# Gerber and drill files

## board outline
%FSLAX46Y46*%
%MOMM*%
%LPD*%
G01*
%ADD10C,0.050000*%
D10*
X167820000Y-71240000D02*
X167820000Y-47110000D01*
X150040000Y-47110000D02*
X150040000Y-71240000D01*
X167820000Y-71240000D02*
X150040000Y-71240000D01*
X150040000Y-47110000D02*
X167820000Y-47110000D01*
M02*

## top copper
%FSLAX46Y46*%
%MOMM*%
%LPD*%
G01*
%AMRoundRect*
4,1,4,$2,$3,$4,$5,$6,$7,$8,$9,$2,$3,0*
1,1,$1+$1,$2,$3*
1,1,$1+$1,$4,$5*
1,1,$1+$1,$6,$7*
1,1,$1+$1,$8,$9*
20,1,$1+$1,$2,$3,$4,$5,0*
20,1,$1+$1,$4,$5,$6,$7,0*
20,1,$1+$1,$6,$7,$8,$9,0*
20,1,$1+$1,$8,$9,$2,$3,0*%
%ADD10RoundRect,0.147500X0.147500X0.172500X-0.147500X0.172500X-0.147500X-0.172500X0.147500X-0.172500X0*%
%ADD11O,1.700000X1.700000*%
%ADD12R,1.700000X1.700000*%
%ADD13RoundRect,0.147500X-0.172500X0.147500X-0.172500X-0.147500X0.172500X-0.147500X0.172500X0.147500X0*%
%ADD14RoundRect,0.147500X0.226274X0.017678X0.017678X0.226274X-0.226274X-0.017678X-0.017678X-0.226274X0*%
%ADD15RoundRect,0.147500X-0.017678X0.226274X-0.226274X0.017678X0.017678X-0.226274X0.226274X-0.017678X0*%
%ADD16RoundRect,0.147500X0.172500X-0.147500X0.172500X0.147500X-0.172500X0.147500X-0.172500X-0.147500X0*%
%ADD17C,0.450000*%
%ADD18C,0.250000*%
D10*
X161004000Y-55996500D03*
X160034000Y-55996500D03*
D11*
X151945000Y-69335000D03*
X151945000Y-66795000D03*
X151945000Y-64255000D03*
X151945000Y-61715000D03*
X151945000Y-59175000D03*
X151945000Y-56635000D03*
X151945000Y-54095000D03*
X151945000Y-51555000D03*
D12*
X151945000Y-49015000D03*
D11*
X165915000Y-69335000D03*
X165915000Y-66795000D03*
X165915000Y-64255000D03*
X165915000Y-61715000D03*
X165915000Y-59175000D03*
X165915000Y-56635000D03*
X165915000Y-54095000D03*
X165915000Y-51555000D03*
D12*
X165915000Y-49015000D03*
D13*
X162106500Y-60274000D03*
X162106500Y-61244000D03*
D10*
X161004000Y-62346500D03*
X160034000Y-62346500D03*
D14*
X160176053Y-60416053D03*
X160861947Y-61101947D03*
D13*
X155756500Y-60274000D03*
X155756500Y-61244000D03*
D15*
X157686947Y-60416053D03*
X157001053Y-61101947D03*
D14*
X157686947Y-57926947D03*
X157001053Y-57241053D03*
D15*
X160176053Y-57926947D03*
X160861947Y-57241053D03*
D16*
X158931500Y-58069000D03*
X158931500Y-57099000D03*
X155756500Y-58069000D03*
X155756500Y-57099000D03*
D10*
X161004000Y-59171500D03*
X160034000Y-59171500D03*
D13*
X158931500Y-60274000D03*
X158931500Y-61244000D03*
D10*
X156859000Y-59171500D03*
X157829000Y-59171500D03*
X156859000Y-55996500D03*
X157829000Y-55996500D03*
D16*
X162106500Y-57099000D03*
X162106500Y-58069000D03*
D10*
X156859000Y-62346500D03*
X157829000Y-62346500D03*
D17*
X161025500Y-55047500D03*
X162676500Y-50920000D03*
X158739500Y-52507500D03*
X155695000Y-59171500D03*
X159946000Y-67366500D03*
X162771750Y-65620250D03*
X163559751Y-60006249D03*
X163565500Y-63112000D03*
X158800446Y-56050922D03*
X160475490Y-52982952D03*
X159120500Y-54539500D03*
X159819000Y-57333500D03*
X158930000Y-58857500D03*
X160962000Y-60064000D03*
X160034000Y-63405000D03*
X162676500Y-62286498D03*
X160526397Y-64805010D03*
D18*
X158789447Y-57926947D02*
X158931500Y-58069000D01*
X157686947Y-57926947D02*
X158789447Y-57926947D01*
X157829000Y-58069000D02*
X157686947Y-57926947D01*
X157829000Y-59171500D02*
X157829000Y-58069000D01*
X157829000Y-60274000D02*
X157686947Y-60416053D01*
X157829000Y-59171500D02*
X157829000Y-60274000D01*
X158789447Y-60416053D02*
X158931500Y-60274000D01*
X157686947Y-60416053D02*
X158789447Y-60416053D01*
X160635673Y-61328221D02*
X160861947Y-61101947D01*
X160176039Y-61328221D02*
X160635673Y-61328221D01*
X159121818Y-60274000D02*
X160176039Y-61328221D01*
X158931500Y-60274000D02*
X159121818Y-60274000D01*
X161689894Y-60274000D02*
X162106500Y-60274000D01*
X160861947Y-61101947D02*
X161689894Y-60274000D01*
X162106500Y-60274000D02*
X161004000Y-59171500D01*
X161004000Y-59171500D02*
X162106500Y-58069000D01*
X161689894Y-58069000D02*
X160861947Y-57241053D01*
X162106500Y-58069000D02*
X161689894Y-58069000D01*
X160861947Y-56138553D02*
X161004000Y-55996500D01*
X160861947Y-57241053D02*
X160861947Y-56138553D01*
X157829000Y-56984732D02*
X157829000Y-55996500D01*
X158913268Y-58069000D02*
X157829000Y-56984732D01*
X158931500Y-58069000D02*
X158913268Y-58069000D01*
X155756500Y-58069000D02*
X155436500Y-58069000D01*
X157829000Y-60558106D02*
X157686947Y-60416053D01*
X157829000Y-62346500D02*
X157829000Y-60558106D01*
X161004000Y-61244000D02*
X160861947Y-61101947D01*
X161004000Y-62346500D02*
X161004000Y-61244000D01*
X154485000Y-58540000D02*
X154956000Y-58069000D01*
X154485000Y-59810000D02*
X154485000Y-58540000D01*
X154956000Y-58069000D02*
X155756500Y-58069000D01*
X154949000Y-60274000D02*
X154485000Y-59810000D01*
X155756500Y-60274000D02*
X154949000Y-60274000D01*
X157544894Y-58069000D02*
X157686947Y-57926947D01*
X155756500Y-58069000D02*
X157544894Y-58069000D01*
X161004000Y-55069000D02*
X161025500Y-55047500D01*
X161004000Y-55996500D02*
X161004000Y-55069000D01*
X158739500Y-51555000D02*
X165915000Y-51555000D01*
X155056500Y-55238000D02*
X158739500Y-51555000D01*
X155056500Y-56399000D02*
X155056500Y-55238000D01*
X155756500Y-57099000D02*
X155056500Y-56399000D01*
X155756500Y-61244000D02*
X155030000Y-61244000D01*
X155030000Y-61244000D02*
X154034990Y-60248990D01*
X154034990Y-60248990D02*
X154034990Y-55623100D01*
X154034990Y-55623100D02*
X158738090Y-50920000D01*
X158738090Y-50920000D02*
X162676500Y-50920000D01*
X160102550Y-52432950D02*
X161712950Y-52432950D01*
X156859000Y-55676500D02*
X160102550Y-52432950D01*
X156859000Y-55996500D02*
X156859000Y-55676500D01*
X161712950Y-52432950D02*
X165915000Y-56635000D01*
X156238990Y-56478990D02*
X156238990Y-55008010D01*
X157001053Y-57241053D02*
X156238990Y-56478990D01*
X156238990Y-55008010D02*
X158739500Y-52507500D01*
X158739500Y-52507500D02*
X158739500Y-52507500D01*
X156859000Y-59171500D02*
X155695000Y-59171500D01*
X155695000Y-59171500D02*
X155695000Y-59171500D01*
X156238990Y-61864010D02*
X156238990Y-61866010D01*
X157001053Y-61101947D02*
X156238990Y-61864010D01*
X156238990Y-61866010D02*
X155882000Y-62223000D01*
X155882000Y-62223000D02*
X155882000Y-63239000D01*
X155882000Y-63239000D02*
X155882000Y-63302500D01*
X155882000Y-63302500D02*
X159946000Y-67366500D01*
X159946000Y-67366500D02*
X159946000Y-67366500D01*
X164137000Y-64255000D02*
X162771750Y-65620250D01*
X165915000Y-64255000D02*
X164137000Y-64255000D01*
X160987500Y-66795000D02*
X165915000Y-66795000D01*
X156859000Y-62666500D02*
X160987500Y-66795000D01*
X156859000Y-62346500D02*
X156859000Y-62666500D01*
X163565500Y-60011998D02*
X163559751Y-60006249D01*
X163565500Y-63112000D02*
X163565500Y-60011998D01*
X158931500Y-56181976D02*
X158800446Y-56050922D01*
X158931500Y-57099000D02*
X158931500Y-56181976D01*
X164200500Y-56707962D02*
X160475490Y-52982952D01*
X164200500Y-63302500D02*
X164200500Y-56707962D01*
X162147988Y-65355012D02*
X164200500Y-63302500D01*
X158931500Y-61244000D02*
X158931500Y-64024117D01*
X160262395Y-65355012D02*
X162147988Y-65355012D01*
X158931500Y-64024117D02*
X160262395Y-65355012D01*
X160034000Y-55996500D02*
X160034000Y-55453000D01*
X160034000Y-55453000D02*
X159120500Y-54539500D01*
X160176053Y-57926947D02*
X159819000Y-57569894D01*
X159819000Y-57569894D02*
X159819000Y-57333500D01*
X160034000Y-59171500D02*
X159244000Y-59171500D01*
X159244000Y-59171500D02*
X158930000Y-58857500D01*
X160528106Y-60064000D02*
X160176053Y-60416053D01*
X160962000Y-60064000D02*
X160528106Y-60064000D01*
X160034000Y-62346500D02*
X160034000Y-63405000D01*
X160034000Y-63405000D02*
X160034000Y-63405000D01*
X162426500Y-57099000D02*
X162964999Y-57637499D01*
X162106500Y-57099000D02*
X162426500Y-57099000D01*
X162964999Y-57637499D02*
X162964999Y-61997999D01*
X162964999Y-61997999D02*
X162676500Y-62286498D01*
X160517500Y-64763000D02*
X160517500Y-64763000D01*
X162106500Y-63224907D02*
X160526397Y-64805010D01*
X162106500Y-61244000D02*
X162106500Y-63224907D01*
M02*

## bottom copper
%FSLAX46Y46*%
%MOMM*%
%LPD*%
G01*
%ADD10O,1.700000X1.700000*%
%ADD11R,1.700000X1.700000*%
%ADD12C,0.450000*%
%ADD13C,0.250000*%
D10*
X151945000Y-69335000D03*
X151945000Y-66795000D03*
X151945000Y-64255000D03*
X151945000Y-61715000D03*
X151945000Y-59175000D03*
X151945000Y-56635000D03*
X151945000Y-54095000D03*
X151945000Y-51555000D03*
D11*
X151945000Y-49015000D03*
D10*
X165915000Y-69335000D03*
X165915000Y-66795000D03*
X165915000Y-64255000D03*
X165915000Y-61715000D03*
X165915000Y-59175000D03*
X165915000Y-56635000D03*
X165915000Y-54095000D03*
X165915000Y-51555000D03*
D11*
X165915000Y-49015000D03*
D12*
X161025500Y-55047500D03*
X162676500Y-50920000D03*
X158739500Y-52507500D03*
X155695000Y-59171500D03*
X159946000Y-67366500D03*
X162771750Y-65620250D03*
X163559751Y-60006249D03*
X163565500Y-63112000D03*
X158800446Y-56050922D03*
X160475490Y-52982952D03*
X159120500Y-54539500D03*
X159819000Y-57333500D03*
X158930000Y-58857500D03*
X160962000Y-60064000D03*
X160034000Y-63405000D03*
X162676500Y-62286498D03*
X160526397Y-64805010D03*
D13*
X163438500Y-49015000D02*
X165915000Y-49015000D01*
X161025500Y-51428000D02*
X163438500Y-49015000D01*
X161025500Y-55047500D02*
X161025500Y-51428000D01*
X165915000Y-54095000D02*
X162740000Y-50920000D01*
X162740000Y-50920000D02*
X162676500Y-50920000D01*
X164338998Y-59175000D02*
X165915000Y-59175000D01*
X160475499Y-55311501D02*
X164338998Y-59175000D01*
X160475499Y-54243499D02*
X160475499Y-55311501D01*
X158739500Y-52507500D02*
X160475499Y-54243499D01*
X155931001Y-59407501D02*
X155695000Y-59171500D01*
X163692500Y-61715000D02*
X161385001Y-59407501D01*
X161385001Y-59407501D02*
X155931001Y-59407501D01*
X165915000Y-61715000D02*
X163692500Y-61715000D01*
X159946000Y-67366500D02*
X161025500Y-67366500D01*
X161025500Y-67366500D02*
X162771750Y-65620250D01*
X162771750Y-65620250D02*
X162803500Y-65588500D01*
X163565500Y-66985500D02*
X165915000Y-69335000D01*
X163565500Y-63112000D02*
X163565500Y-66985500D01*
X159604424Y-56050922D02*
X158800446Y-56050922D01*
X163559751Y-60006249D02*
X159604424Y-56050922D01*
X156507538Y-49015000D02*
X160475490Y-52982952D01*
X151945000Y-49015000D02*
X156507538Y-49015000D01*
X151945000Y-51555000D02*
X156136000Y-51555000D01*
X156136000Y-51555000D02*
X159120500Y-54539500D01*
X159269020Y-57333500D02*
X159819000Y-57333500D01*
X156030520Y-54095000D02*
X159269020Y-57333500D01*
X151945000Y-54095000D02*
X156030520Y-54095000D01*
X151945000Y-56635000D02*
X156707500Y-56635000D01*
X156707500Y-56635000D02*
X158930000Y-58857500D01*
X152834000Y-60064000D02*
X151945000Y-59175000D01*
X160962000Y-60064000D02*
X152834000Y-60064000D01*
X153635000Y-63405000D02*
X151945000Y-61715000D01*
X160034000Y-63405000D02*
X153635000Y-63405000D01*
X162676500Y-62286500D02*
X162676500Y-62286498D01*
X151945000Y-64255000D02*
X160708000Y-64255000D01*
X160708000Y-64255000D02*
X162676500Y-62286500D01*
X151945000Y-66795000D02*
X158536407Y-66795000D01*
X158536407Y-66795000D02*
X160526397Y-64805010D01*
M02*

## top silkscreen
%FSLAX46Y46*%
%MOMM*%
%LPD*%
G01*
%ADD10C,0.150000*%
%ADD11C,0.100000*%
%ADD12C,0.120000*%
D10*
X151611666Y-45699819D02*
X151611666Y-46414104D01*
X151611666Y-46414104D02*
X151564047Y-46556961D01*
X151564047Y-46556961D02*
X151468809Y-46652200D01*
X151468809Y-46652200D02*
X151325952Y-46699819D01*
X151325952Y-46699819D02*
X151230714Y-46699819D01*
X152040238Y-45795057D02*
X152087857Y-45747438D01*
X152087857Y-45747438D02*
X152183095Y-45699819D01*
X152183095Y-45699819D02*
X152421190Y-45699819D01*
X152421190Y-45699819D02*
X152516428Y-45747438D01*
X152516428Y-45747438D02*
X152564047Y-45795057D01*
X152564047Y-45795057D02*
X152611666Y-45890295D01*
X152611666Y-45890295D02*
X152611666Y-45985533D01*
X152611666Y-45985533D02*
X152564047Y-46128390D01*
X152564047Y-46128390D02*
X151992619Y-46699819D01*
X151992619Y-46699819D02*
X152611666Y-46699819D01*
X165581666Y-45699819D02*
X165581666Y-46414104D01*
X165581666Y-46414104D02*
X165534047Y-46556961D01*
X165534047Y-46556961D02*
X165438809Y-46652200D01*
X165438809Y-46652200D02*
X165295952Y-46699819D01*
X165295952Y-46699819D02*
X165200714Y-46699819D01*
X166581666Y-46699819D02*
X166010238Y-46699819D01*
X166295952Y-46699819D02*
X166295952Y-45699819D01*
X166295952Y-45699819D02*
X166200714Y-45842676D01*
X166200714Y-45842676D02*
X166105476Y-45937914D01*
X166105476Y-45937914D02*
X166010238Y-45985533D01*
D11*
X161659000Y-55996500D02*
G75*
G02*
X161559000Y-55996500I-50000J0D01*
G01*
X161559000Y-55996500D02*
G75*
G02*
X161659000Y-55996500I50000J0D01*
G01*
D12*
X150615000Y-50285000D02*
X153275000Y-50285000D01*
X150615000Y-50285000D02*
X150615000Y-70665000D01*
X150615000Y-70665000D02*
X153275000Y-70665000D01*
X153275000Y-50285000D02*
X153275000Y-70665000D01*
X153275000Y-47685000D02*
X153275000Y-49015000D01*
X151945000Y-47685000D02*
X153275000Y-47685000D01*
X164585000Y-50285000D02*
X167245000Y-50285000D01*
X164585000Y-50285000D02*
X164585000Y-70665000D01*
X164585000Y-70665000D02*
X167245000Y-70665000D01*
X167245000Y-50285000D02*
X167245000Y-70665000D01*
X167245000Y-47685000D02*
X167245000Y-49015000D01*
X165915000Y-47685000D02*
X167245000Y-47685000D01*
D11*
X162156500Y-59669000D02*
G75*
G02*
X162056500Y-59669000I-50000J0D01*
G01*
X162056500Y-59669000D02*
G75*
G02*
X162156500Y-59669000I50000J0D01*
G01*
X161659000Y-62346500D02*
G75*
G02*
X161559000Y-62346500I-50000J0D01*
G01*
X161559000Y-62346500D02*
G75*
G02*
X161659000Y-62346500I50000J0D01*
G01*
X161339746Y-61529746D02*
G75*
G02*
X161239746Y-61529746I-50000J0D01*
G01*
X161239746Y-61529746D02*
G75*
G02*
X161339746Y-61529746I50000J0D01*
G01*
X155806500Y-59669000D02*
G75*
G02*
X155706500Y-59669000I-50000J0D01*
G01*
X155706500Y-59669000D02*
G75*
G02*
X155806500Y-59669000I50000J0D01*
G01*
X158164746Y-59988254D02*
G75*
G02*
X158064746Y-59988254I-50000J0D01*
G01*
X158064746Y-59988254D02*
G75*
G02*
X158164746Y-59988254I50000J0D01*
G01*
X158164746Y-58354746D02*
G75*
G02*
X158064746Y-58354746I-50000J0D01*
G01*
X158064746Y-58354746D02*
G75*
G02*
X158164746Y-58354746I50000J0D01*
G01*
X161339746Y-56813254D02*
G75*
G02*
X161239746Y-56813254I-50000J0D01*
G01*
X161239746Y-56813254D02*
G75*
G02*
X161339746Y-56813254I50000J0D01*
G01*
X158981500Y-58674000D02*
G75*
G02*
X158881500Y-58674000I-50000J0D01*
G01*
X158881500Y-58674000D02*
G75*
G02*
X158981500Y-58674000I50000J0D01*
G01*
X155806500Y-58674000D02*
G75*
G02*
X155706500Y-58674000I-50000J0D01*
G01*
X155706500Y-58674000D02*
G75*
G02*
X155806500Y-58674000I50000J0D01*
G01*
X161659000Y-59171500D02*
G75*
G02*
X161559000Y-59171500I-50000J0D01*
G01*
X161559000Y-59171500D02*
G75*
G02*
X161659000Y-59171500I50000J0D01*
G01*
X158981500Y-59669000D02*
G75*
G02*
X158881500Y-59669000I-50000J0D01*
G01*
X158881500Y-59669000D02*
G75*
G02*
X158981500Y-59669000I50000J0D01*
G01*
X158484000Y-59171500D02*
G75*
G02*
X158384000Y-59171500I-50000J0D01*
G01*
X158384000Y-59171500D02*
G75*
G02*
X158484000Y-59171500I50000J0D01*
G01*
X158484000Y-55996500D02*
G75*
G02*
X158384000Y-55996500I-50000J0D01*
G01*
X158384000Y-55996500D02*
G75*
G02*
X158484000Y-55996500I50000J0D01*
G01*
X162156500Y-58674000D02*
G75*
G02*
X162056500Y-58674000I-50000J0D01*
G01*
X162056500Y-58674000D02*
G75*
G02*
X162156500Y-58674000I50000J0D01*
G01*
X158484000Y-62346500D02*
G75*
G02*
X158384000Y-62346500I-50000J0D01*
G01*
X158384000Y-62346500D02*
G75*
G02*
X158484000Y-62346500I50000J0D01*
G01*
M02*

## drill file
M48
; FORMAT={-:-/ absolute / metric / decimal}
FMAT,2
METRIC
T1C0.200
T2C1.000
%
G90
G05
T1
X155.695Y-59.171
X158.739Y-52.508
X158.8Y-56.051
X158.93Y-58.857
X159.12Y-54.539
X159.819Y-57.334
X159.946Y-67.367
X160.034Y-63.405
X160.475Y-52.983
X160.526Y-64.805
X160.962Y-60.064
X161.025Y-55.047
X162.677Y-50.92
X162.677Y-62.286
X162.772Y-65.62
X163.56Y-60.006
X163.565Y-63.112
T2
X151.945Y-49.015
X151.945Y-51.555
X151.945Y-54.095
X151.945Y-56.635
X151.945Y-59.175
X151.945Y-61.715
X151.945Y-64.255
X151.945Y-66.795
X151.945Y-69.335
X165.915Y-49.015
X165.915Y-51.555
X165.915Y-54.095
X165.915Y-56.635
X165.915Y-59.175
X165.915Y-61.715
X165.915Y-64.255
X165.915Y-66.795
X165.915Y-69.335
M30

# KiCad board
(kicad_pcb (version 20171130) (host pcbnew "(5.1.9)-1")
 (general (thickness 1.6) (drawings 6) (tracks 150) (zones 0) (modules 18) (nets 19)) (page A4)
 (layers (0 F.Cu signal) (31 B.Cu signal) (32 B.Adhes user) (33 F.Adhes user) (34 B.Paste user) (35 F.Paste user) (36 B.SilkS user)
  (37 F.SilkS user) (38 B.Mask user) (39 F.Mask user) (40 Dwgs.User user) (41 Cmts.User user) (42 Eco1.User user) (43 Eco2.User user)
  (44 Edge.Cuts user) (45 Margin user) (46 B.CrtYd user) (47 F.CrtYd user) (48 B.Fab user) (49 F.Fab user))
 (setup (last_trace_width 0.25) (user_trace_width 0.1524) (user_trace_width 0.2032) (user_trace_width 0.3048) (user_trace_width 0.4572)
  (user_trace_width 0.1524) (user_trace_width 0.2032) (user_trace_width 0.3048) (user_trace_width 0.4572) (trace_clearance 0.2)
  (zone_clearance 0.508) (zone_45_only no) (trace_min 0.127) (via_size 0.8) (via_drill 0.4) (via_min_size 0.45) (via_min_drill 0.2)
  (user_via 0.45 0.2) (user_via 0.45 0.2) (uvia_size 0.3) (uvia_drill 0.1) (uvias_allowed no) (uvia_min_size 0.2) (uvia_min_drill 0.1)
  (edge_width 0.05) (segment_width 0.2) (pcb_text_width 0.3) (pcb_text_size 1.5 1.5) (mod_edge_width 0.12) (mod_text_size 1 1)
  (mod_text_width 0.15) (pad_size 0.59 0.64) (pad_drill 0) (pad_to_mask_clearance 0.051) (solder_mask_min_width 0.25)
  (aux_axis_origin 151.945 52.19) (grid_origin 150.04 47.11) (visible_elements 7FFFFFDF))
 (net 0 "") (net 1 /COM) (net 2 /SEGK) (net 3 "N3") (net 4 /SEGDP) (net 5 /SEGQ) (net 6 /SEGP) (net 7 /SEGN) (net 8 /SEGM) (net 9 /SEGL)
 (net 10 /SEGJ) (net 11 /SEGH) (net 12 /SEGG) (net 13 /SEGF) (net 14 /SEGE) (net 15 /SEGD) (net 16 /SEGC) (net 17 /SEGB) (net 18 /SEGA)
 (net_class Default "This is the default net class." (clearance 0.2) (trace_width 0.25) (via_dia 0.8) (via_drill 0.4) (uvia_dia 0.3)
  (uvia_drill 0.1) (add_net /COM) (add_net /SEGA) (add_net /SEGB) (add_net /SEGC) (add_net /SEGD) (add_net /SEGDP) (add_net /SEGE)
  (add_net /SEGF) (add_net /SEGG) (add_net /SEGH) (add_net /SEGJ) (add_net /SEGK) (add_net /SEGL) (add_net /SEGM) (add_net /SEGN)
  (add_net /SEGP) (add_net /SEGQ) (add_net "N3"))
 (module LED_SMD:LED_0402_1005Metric (layer F.Cu) (at 160.519 55.9965 180)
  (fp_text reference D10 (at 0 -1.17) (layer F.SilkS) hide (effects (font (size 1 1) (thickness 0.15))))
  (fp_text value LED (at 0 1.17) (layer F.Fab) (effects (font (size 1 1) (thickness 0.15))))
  (fp_circle (center -1.09 0) (end -1.04 0) (layer F.SilkS) (width 0.1))
  (pad 1 smd roundrect (at -0.485 0 180) (size 0.59 0.64) (layers F.Cu F.Paste F.Mask) (roundrect_rratio 0.25) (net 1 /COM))
  (pad 2 smd roundrect (at 0.485 0 180) (size 0.59 0.64) (layers F.Cu F.Paste F.Mask) (roundrect_rratio 0.25) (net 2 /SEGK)))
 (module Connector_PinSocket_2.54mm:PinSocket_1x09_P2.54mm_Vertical (layer F.Cu) (at 151.945 49.015)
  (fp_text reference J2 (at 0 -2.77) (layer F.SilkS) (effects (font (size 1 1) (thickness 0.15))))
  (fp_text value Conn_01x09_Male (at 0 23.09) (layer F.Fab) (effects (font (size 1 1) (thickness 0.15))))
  (fp_line (start -1.33 1.27) (end 1.33 1.27) (layer F.SilkS) (width 0.12))
  (fp_line (start -1.33 1.27) (end -1.33 21.65) (layer F.SilkS) (width 0.12))
  (fp_line (start -1.33 21.65) (end 1.33 21.65) (layer F.SilkS) (width 0.12))
  (fp_line (start 1.33 1.27) (end 1.33 21.65) (layer F.SilkS) (width 0.12))
  (fp_line (start 1.33 -1.33) (end 1.33 0) (layer F.SilkS) (width 0.12))
  (fp_line (start 0 -1.33) (end 1.33 -1.33) (layer F.SilkS) (width 0.12))
  (pad 9 thru_hole oval (at 0 20.32) (size 1.7 1.7) (drill 1) (layers *.Cu *.Mask) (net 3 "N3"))
  (pad 8 thru_hole oval (at 0 17.78) (size 1.7 1.7) (drill 1) (layers *.Cu *.Mask) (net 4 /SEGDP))
  (pad 7 thru_hole oval (at 0 15.24) (size 1.7 1.7) (drill 1) (layers *.Cu *.Mask) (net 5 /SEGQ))
  (pad 6 thru_hole oval (at 0 12.7) (size 1.7 1.7) (drill 1) (layers *.Cu *.Mask) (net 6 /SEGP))
  (pad 5 thru_hole oval (at 0 10.16) (size 1.7 1.7) (drill 1) (layers *.Cu *.Mask) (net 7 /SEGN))
  (pad 4 thru_hole oval (at 0 7.62) (size 1.7 1.7) (drill 1) (layers *.Cu *.Mask) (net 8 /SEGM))
  (pad 3 thru_hole oval (at 0 5.08) (size 1.7 1.7) (drill 1) (layers *.Cu *.Mask) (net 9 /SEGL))
  (pad 2 thru_hole oval (at 0 2.54) (size 1.7 1.7) (drill 1) (layers *.Cu *.Mask) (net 2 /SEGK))
  (pad 1 thru_hole rect (at 0 0) (size 1.7 1.7) (drill 1) (layers *.Cu *.Mask) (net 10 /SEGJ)))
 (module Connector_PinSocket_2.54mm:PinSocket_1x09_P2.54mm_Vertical (layer F.Cu) (at 165.915 49.015)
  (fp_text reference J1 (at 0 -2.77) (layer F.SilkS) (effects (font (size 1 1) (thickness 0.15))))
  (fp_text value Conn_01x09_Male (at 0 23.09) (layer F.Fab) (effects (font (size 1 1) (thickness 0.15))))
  (fp_line (start -1.33 1.27) (end 1.33 1.27) (layer F.SilkS) (width 0.12))
  (fp_line (start -1.33 1.27) (end -1.33 21.65) (layer F.SilkS) (width 0.12))
  (fp_line (start -1.33 21.65) (end 1.33 21.65) (layer F.SilkS) (width 0.12))
  (fp_line (start 1.33 1.27) (end 1.33 21.65) (layer F.SilkS) (width 0.12))
  (fp_line (start 1.33 -1.33) (end 1.33 0) (layer F.SilkS) (width 0.12))
  (fp_line (start 0 -1.33) (end 1.33 -1.33) (layer F.SilkS) (width 0.12))
  (pad 9 thru_hole oval (at 0 20.32) (size 1.7 1.7) (drill 1) (layers *.Cu *.Mask) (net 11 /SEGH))
  (pad 8 thru_hole oval (at 0 17.78) (size 1.7 1.7) (drill 1) (layers *.Cu *.Mask) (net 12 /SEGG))
  (pad 7 thru_hole oval (at 0 15.24) (size 1.7 1.7) (drill 1) (layers *.Cu *.Mask) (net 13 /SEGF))
  (pad 6 thru_hole oval (at 0 12.7) (size 1.7 1.7) (drill 1) (layers *.Cu *.Mask) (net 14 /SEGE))
  (pad 5 thru_hole oval (at 0 10.16) (size 1.7 1.7) (drill 1) (layers *.Cu *.Mask) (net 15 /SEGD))
  (pad 4 thru_hole oval (at 0 7.62) (size 1.7 1.7) (drill 1) (layers *.Cu *.Mask) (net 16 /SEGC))
  (pad 3 thru_hole oval (at 0 5.08) (size 1.7 1.7) (drill 1) (layers *.Cu *.Mask) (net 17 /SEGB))
  (pad 2 thru_hole oval (at 0 2.54) (size 1.7 1.7) (drill 1) (layers *.Cu *.Mask) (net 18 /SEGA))
  (pad 1 thru_hole rect (at 0 0) (size 1.7 1.7) (drill 1) (layers *.Cu *.Mask) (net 1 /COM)))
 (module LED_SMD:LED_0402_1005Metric (layer F.Cu) (at 162.1065 60.759 270)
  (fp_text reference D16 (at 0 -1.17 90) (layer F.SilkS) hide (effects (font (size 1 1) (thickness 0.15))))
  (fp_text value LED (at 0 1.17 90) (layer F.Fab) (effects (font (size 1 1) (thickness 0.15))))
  (fp_circle (center -1.09 0) (end -1.04 0) (layer F.SilkS) (width 0.1))
  (pad 1 smd roundrect (at -0.485 0 270) (size 0.59 0.64) (layers F.Cu F.Paste F.Mask) (roundrect_rratio 0.25) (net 1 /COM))
  (pad 2 smd roundrect (at 0.485 0 270) (size 0.59 0.64) (layers F.Cu F.Paste F.Mask) (roundrect_rratio 0.25) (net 4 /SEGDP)))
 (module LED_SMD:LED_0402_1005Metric (layer F.Cu) (at 160.519 62.3465 180)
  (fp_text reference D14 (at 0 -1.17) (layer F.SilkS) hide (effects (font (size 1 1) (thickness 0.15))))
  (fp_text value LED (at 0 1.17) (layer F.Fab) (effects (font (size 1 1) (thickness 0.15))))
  (fp_circle (center -1.09 0) (end -1.04 0) (layer F.SilkS) (width 0.1))
  (pad 1 smd roundrect (at -0.485 0 180) (size 0.59 0.64) (layers F.Cu F.Paste F.Mask) (roundrect_rratio 0.25) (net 1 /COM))
  (pad 2 smd roundrect (at 0.485 0 180) (size 0.59 0.64) (layers F.Cu F.Paste F.Mask) (roundrect_rratio 0.25) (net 6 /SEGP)))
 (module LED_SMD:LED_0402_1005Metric (layer F.Cu) (at 160.519 60.759 135)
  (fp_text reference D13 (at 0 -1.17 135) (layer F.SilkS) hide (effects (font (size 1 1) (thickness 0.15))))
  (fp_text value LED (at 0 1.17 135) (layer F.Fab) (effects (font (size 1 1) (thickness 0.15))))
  (fp_circle (center -1.09 0) (end -1.04 0) (layer F.SilkS) (width 0.1))
  (pad 2 smd roundrect (at 0.485 0 135) (size 0.59 0.64) (layers F.Cu F.Paste F.Mask) (roundrect_rratio 0.25) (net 7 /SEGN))
  (pad 1 smd roundrect (at -0.485 0 135) (size 0.59 0.64) (layers F.Cu F.Paste F.Mask) (roundrect_rratio 0.25) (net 1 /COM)))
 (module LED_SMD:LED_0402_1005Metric (layer F.Cu) (at 155.7565 60.759 270)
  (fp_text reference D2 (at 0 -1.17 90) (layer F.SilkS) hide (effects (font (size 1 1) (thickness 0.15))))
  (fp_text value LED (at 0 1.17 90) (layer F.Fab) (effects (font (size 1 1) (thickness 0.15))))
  (fp_circle (center -1.09 0) (end -1.04 0) (layer F.SilkS) (width 0.1))
  (pad 1 smd roundrect (at -0.485 0 270) (size 0.59 0.64) (layers F.Cu F.Paste F.Mask) (roundrect_rratio 0.25) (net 1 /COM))
  (pad 2 smd roundrect (at 0.485 0 270) (size 0.59 0.64) (layers F.Cu F.Paste F.Mask) (roundrect_rratio 0.25) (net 17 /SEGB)))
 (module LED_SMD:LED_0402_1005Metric (layer F.Cu) (at 157.344 60.759 225)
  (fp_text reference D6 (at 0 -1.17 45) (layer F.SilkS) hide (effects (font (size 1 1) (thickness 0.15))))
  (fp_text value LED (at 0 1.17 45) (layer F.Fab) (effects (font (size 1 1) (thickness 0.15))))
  (fp_circle (center -1.09 0) (end -1.04 0) (layer F.SilkS) (width 0.1))
  (pad 1 smd roundrect (at -0.485 0 225) (size 0.59 0.64) (layers F.Cu F.Paste F.Mask) (roundrect_rratio 0.25) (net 1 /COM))
  (pad 2 smd roundrect (at 0.485 0 225) (size 0.59 0.64) (layers F.Cu F.Paste F.Mask) (roundrect_rratio 0.25) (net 13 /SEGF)))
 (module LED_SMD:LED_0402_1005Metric (layer F.Cu) (at 157.344 57.584 135)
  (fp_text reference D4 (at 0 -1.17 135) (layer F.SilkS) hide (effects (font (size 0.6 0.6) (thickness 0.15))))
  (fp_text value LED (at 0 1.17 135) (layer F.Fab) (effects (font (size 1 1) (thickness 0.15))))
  (fp_circle (center -1.09 0) (end -1.04 0) (layer F.SilkS) (width 0.1))
  (pad 1 smd roundrect (at -0.485 0 135) (size 0.59 0.64) (layers F.Cu F.Paste F.Mask) (roundrect_rratio 0.25) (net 1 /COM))
  (pad 2 smd roundrect (at 0.485 0 135) (size 0.59 0.64) (layers F.Cu F.Paste F.Mask) (roundrect_rratio 0.25) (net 15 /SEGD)))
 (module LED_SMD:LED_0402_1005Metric (layer F.Cu) (at 160.519 57.584 225)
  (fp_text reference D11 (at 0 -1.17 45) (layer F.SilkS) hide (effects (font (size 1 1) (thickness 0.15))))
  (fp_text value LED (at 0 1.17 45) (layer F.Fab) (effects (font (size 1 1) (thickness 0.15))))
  (fp_circle (center -1.09 0) (end -1.04 0) (layer F.SilkS) (width 0.1))
  (pad 2 smd roundrect (at 0.485 0 225) (size 0.59 0.64) (layers F.Cu F.Paste F.Mask) (roundrect_rratio 0.25) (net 9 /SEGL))
  (pad 1 smd roundrect (at -0.485 0 225) (size 0.59 0.64) (layers F.Cu F.Paste F.Mask) (roundrect_rratio 0.25) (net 1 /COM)))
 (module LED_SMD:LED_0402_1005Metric (layer F.Cu) (at 158.9315 57.584 90)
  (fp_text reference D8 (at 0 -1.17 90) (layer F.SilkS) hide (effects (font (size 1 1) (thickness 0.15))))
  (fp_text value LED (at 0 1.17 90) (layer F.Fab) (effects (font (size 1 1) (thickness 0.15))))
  (fp_circle (center -1.09 0) (end -1.04 0) (layer F.SilkS) (width 0.1))
  (pad 1 smd roundrect (at -0.485 0 90) (size 0.59 0.64) (layers F.Cu F.Paste F.Mask) (roundrect_rratio 0.25) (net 1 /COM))
  (pad 2 smd roundrect (at 0.485 0 90) (size 0.59 0.64) (layers F.Cu F.Paste F.Mask) (roundrect_rratio 0.25) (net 11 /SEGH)))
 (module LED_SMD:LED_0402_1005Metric (layer F.Cu) (at 155.7565 57.584 90)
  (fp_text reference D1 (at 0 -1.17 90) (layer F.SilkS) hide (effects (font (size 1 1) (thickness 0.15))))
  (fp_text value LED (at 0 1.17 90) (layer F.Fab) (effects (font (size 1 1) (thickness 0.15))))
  (fp_circle (center -1.09 0) (end -1.04 0) (layer F.SilkS) (width 0.1))
  (pad 1 smd roundrect (at -0.485 0 90) (size 0.59 0.64) (layers F.Cu F.Paste F.Mask) (roundrect_rratio 0.25) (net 1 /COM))
  (pad 2 smd roundrect (at 0.485 0 90) (size 0.59 0.64) (layers F.Cu F.Paste F.Mask) (roundrect_rratio 0.25) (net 18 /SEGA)))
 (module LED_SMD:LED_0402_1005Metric (layer F.Cu) (at 160.519 59.1715 180)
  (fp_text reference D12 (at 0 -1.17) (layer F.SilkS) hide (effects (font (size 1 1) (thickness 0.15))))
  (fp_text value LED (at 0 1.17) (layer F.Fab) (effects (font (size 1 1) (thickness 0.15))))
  (fp_circle (center -1.09 0) (end -1.04 0) (layer F.SilkS) (width 0.1))
  (pad 1 smd roundrect (at -0.485 0 180) (size 0.59 0.64) (layers F.Cu F.Paste F.Mask) (roundrect_rratio 0.25) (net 1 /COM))
  (pad 2 smd roundrect (at 0.485 0 180) (size 0.59 0.64) (layers F.Cu F.Paste F.Mask) (roundrect_rratio 0.25) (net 8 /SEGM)))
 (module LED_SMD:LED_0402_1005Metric (layer F.Cu) (at 158.9315 60.759 270)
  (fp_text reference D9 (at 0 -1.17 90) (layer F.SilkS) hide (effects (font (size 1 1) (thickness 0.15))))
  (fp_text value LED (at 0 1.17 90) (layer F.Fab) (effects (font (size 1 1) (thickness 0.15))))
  (fp_circle (center -1.09 0) (end -1.04 0) (layer F.SilkS) (width 0.1))
  (pad 1 smd roundrect (at -0.485 0 270) (size 0.59 0.64) (layers F.Cu F.Paste F.Mask) (roundrect_rratio 0.25) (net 1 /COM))
  (pad 2 smd roundrect (at 0.485 0 270) (size 0.59 0.64) (layers F.Cu F.Paste F.Mask) (roundrect_rratio 0.25) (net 10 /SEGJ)))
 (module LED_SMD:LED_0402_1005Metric (layer F.Cu) (at 157.344 59.1715 180)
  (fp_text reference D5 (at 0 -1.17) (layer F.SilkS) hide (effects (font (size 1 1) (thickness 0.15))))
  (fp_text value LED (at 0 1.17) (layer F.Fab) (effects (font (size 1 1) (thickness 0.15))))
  (fp_circle (center -1.09 0) (end -1.04 0) (layer F.SilkS) (width 0.1))
  (pad 2 smd roundrect (at 0.485 0 180) (size 0.59 0.64) (layers F.Cu F.Paste F.Mask) (roundrect_rratio 0.25) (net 14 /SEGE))
  (pad 1 smd roundrect (at -0.485 0 180) (size 0.59 0.64) (layers F.Cu F.Paste F.Mask) (roundrect_rratio 0.25) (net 1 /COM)))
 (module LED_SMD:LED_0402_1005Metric (layer F.Cu) (at 157.344 55.9965 180)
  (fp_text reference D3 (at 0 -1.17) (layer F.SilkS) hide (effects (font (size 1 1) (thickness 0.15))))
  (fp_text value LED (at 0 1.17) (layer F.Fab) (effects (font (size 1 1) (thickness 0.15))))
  (fp_circle (center -1.09 0) (end -1.04 0) (layer F.SilkS) (width 0.1))
  (pad 2 smd roundrect (at 0.485 0 180) (size 0.59 0.64) (layers F.Cu F.Paste F.Mask) (roundrect_rratio 0.25) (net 16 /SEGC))
  (pad 1 smd roundrect (at -0.485 0 180) (size 0.59 0.64) (layers F.Cu F.Paste F.Mask) (roundrect_rratio 0.25) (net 1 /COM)))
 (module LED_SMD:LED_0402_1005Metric (layer F.Cu) (at 162.1065 57.584 90)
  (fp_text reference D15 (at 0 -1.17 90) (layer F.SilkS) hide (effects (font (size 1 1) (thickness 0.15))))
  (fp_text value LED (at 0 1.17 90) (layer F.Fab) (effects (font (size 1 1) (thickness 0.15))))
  (fp_circle (center -1.09 0) (end -1.04 0) (layer F.SilkS) (width 0.1))
  (pad 2 smd roundrect (at 0.485 0 90) (size 0.59 0.64) (layers F.Cu F.Paste F.Mask) (roundrect_rratio 0.25) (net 5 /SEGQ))
  (pad 1 smd roundrect (at -0.485 0 90) (size 0.59 0.64) (layers F.Cu F.Paste F.Mask) (roundrect_rratio 0.25) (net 1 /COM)))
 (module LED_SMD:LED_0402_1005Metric (layer F.Cu) (at 157.344 62.3465 180)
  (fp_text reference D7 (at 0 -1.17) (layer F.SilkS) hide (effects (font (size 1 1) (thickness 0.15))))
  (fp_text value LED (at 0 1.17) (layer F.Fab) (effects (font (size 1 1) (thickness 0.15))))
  (fp_circle (center -1.09 0) (end -1.04 0) (layer F.SilkS) (width 0.1))
  (pad 2 smd roundrect (at 0.485 0 180) (size 0.59 0.64) (layers F.Cu F.Paste F.Mask) (roundrect_rratio 0.25) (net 12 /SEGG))
  (pad 1 smd roundrect (at -0.485 0 180) (size 0.59 0.64) (layers F.Cu F.Paste F.Mask) (roundrect_rratio 0.25) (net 1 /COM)))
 (gr_line (start 167.82 71.24) (end 167.82 47.11) (layer Edge.Cuts) (width 0.05))
 (gr_line (start 150.04 47.11) (end 150.04 71.24) (layer Edge.Cuts) (width 0.05))
 (gr_line (start 167.82 71.24) (end 150.04 71.24) (layer Edge.Cuts) (width 0.05))
 (gr_line (start 150.04 47.11) (end 167.82 47.11) (layer Edge.Cuts) (width 0.05))
 (via (at 161.0255 55.0475) (size 0.45) (drill 0.2) (layers F.Cu B.Cu) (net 1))
 (segment (start 158.789447 57.926947) (end 158.9315 58.069) (width 0.25) (layer F.Cu) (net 1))
 (segment (start 157.686947 57.926947) (end 158.789447 57.926947) (width 0.25) (layer F.Cu) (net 1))
 (segment (start 157.829 58.069) (end 157.686947 57.926947) (width 0.25) (layer F.Cu) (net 1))
 (segment (start 157.829 59.1715) (end 157.829 58.069) (width 0.25) (layer F.Cu) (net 1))
 (segment (start 157.829 60.274) (end 157.686947 60.416053) (width 0.25) (layer F.Cu) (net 1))
 (segment (start 157.829 59.1715) (end 157.829 60.274) (width 0.25) (layer F.Cu) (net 1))
 (segment (start 158.789447 60.416053) (end 158.9315 60.274) (width 0.25) (layer F.Cu) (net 1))
 (segment (start 157.686947 60.416053) (end 158.789447 60.416053) (width 0.25) (layer F.Cu) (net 1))
 (segment (start 160.635673 61.328221) (end 160.861947 61.101947) (width 0.25) (layer F.Cu) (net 1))
 (segment (start 160.176039 61.328221) (end 160.635673 61.328221) (width 0.25) (layer F.Cu) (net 1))
 (segment (start 159.121818 60.274) (end 160.176039 61.328221) (width 0.25) (layer F.Cu) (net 1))
 (segment (start 158.9315 60.274) (end 159.121818 60.274) (width 0.25) (layer F.Cu) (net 1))
 (segment (start 161.689894 60.274) (end 162.1065 60.274) (width 0.25) (layer F.Cu) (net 1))
 (segment (start 160.861947 61.101947) (end 161.689894 60.274) (width 0.25) (layer F.Cu) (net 1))
 (segment (start 162.1065 60.274) (end 161.004 59.1715) (width 0.25) (layer F.Cu) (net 1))
 (segment (start 161.004 59.1715) (end 162.1065 58.069) (width 0.25) (layer F.Cu) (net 1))
 (segment (start 161.689894 58.069) (end 160.861947 57.241053) (width 0.25) (layer F.Cu) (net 1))
 (segment (start 162.1065 58.069) (end 161.689894 58.069) (width 0.25) (layer F.Cu) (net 1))
 (segment (start 160.861947 56.138553) (end 161.004 55.9965) (width 0.25) (layer F.Cu) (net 1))
 (segment (start 160.861947 57.241053) (end 160.861947 56.138553) (width 0.25) (layer F.Cu) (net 1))
 (segment (start 157.829 56.984732) (end 157.829 55.9965) (width 0.25) (layer F.Cu) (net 1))
 (segment (start 158.913268 58.069) (end 157.829 56.984732) (width 0.25) (layer F.Cu) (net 1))
 (segment (start 158.9315 58.069) (end 158.913268 58.069) (width 0.25) (layer F.Cu) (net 1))
 (segment (start 155.7565 58.069) (end 155.4365 58.069) (width 0.25) (layer F.Cu) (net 1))
 (segment (start 157.829 60.558106) (end 157.686947 60.416053) (width 0.25) (layer F.Cu) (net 1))
 (segment (start 157.829 62.3465) (end 157.829 60.558106) (width 0.25) (layer F.Cu) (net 1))
 (segment (start 161.004 61.244) (end 160.861947 61.101947) (width 0.25) (layer F.Cu) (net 1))
 (segment (start 161.004 62.3465) (end 161.004 61.244) (width 0.25) (layer F.Cu) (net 1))
 (segment (start 154.485 58.54) (end 154.956 58.069) (width 0.25) (layer F.Cu) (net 1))
 (segment (start 154.485 59.81) (end 154.485 58.54) (width 0.25) (layer F.Cu) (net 1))
 (segment (start 154.956 58.069) (end 155.7565 58.069) (width 0.25) (layer F.Cu) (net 1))
 (segment (start 154.949 60.274) (end 154.485 59.81) (width 0.25) (layer F.Cu) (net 1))
 (segment (start 155.7565 60.274) (end 154.949 60.274) (width 0.25) (layer F.Cu) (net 1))
 (segment (start 157.544894 58.069) (end 157.686947 57.926947) (width 0.25) (layer F.Cu) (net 1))
 (segment (start 155.7565 58.069) (end 157.544894 58.069) (width 0.25) (layer F.Cu) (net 1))
 (segment (start 161.004 55.069) (end 161.0255 55.0475) (width 0.25) (layer F.Cu) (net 1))
 (segment (start 161.004 55.9965) (end 161.004 55.069) (width 0.25) (layer F.Cu) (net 1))
 (segment (start 163.4385 49.015) (end 165.915 49.015) (width 0.25) (layer B.Cu) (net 1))
 (segment (start 161.0255 51.428) (end 163.4385 49.015) (width 0.25) (layer B.Cu) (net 1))
 (segment (start 161.0255 55.0475) (end 161.0255 51.428) (width 0.25) (layer B.Cu) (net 1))
 (segment (start 158.7395 51.555) (end 165.915 51.555) (width 0.25) (layer F.Cu) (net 18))
 (segment (start 155.0565 55.238) (end 158.7395 51.555) (width 0.25) (layer F.Cu) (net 18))
 (segment (start 155.0565 56.399) (end 155.0565 55.238) (width 0.25) (layer F.Cu) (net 18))
 (segment (start 155.7565 57.099) (end 155.0565 56.399) (width 0.25) (layer F.Cu) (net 18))
 (via (at 162.6765 50.92) (size 0.45) (drill 0.2) (layers F.Cu B.Cu) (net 17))
 (segment (start 165.915 54.095) (end 162.74 50.92) (width 0.25) (layer B.Cu) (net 17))
 (segment (start 162.74 50.92) (end 162.6765 50.92) (width 0.25) (layer B.Cu) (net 17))
 (segment (start 155.7565 61.244) (end 155.03 61.244) (width 0.25) (layer F.Cu) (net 17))
 (segment (start 155.03 61.244) (end 154.03499 60.24899) (width 0.25) (layer F.Cu) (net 17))
 (segment (start 154.03499 60.24899) (end 154.03499 55.6231) (width 0.25) (layer F.Cu) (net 17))
 (segment (start 154.03499 55.6231) (end 158.73809 50.92) (width 0.25) (layer F.Cu) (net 17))
 (segment (start 158.73809 50.92) (end 162.6765 50.92) (width 0.25) (layer F.Cu) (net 17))
 (segment (start 160.10255 52.43295) (end 161.71295 52.43295) (width 0.25) (layer F.Cu) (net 16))
 (segment (start 156.859 55.6765) (end 160.10255 52.43295) (width 0.25) (layer F.Cu) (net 16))
 (segment (start 156.859 55.9965) (end 156.859 55.6765) (width 0.25) (layer F.Cu) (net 16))
 (segment (start 161.71295 52.43295) (end 165.915 56.635) (width 0.25) (layer F.Cu) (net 16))
 (segment (start 156.23899 56.47899) (end 156.23899 55.00801) (width 0.25) (layer F.Cu) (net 15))
 (segment (start 157.001053 57.241053) (end 156.23899 56.47899) (width 0.25) (layer F.Cu) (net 15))
 (segment (start 156.23899 55.00801) (end 158.7395 52.5075) (width 0.25) (layer F.Cu) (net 15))
 (segment (start 158.7395 52.5075) (end 158.7395 52.5075) (width 0.25) (layer F.Cu) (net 15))
 (via (at 158.7395 52.5075) (size 0.45) (drill 0.2) (layers F.Cu B.Cu) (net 15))
 (segment (start 164.338998 59.175) (end 165.915 59.175) (width 0.25) (layer B.Cu) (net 15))
 (segment (start 160.475499 55.311501) (end 164.338998 59.175) (width 0.25) (layer B.Cu) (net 15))
 (segment (start 160.475499 54.243499) (end 160.475499 55.311501) (width 0.25) (layer B.Cu) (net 15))
 (segment (start 158.7395 52.5075) (end 160.475499 54.243499) (width 0.25) (layer B.Cu) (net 15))
 (segment (start 156.859 59.1715) (end 155.695 59.1715) (width 0.25) (layer F.Cu) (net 14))
 (segment (start 155.695 59.1715) (end 155.695 59.1715) (width 0.25) (layer F.Cu) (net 14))
 (via (at 155.695 59.1715) (size 0.45) (drill 0.2) (layers F.Cu B.Cu) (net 14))
 (segment (start 155.931001 59.407501) (end 155.695 59.1715) (width 0.25) (layer B.Cu) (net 14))
 (segment (start 163.6925 61.715) (end 161.385001 59.407501) (width 0.25) (layer B.Cu) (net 14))
 (segment (start 161.385001 59.407501) (end 155.931001 59.407501) (width 0.25) (layer B.Cu) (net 14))
 (segment (start 165.915 61.715) (end 163.6925 61.715) (width 0.25) (layer B.Cu) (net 14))
 (segment (start 156.23899 61.86401) (end 156.23899 61.86601) (width 0.25) (layer F.Cu) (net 13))
 (segment (start 157.001053 61.101947) (end 156.23899 61.86401) (width 0.25) (layer F.Cu) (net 13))
 (segment (start 156.23899 61.86601) (end 155.882 62.223) (width 0.25) (layer F.Cu) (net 13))
 (segment (start 155.882 62.223) (end 155.882 63.239) (width 0.25) (layer F.Cu) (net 13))
 (segment (start 155.882 63.239) (end 155.882 63.3025) (width 0.25) (layer F.Cu) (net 13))
 (segment (start 155.882 63.3025) (end 159.946 67.3665) (width 0.25) (layer F.Cu) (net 13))
 (segment (start 159.946 67.3665) (end 159.946 67.3665) (width 0.25) (layer F.Cu) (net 13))
 (via (at 159.946 67.3665) (size 0.45) (drill 0.2) (layers F.Cu B.Cu) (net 13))
 (segment (start 159.946 67.3665) (end 161.0255 67.3665) (width 0.25) (layer B.Cu) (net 13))
 (segment (start 161.0255 67.3665) (end 162.77175 65.62025) (width 0.25) (layer B.Cu) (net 13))
 (segment (start 162.77175 65.62025) (end 162.8035 65.5885) (width 0.25) (layer B.Cu) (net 13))
 (via (at 162.77175 65.62025) (size 0.45) (drill 0.2) (layers F.Cu B.Cu) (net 13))
 (segment (start 164.137 64.255) (end 162.77175 65.62025) (width 0.25) (layer F.Cu) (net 13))
 (segment (start 165.915 64.255) (end 164.137 64.255) (width 0.25) (layer F.Cu) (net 13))
 (segment (start 160.9875 66.795) (end 165.915 66.795) (width 0.25) (layer F.Cu) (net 12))
 (segment (start 156.859 62.6665) (end 160.9875 66.795) (width 0.25) (layer F.Cu) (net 12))
 (segment (start 156.859 62.3465) (end 156.859 62.6665) (width 0.25) (layer F.Cu) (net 12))
 (segment (start 163.5655 66.9855) (end 165.915 69.335) (width 0.25) (layer B.Cu) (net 11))
 (via (at 163.559751 60.006249) (size 0.45) (drill 0.2) (layers F.Cu B.Cu) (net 11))
 (segment (start 163.5655 63.112) (end 163.5655 66.9855) (width 0.25) (layer B.Cu) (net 11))
 (via (at 163.5655 63.112) (size 0.45) (drill 0.2) (layers F.Cu B.Cu) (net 11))
 (segment (start 163.5655 60.011998) (end 163.559751 60.006249) (width 0.25) (layer F.Cu) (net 11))
 (segment (start 163.5655 63.112) (end 163.5655 60.011998) (width 0.25) (layer F.Cu) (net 11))
 (segment (start 158.9315 56.181976) (end 158.800446 56.050922) (width 0.25) (layer F.Cu) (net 11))
 (segment (start 158.9315 57.099) (end 158.9315 56.181976) (width 0.25) (layer F.Cu) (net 11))
 (via (at 158.800446 56.050922) (size 0.45) (drill 0.2) (layers F.Cu B.Cu) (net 11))
 (segment (start 159.604424 56.050922) (end 158.800446 56.050922) (width 0.25) (layer B.Cu) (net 11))
 (segment (start 163.559751 60.006249) (end 159.604424 56.050922) (width 0.25) (layer B.Cu) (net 11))
 (segment (start 164.2005 56.707962) (end 160.47549 52.982952) (width 0.25) (layer F.Cu) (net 10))
 (segment (start 164.2005 63.3025) (end 164.2005 56.707962) (width 0.25) (layer F.Cu) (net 10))
 (segment (start 162.147988 65.355012) (end 164.2005 63.3025) (width 0.25) (layer F.Cu) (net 10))
 (segment (start 158.9315 61.244) (end 158.9315 64.024117) (width 0.25) (layer F.Cu) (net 10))
 (segment (start 156.507538 49.015) (end 160.47549 52.982952) (width 0.25) (layer B.Cu) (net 10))
 (segment (start 151.945 49.015) (end 156.507538 49.015) (width 0.25) (layer B.Cu) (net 10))
 (via (at 160.47549 52.982952) (size 0.45) (drill 0.2) (layers F.Cu B.Cu) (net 10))
 (segment (start 160.262395 65.355012) (end 162.147988 65.355012) (width 0.25) (layer F.Cu) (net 10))
 (segment (start 158.9315 64.024117) (end 160.262395 65.355012) (width 0.25) (layer F.Cu) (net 10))
 (via (at 159.1205 54.5395) (size 0.45) (drill 0.2) (layers F.Cu B.Cu) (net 2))
 (segment (start 160.034 55.9965) (end 160.034 55.453) (width 0.25) (layer F.Cu) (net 2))
 (segment (start 160.034 55.453) (end 159.1205 54.5395) (width 0.25) (layer F.Cu) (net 2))
 (segment (start 151.945 51.555) (end 156.136 51.555) (width 0.25) (layer B.Cu) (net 2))
 (segment (start 156.136 51.555) (end 159.1205 54.5395) (width 0.25) (layer B.Cu) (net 2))
 (via (at 159.819 57.3335) (size 0.45) (drill 0.2) (layers F.Cu B.Cu) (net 9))
 (segment (start 159.26902 57.3335) (end 159.819 57.3335) (width 0.25) (layer B.Cu) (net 9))
 (segment (start 156.03052 54.095) (end 159.26902 57.3335) (width 0.25) (layer B.Cu) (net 9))
 (segment (start 151.945 54.095) (end 156.03052 54.095) (width 0.25) (layer B.Cu) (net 9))
 (segment (start 160.176053 57.926947) (end 159.819 57.569894) (width 0.25) (layer F.Cu) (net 9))
 (segment (start 159.819 57.569894) (end 159.819 57.3335) (width 0.25) (layer F.Cu) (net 9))
 (via (at 158.93 58.8575) (size 0.45) (drill 0.2) (layers F.Cu B.Cu) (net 8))
 (segment (start 151.945 56.635) (end 156.7075 56.635) (width 0.25) (layer B.Cu) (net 8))
 (segment (start 156.7075 56.635) (end 158.93 58.8575) (width 0.25) (layer B.Cu) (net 8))
 (segment (start 160.034 59.1715) (end 159.244 59.1715) (width 0.25) (layer F.Cu) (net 8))
 (segment (start 159.244 59.1715) (end 158.93 58.8575) (width 0.25) (layer F.Cu) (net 8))
 (via (at 160.962 60.064) (size 0.45) (drill 0.2) (layers F.Cu B.Cu) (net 7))
 (segment (start 160.528106 60.064) (end 160.176053 60.416053) (width 0.25) (layer F.Cu) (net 7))
 (segment (start 160.962 60.064) (end 160.528106 60.064) (width 0.25) (layer F.Cu) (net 7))
 (segment (start 152.834 60.064) (end 151.945 59.175) (width 0.25) (layer B.Cu) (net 7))
 (segment (start 160.962 60.064) (end 152.834 60.064) (width 0.25) (layer B.Cu) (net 7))
 (segment (start 160.034 62.3465) (end 160.034 63.405) (width 0.25) (layer F.Cu) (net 6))
 (segment (start 160.034 63.405) (end 160.034 63.405) (width 0.25) (layer F.Cu) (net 6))
 (via (at 160.034 63.405) (size 0.45) (drill 0.2) (layers F.Cu B.Cu) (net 6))
 (segment (start 153.635 63.405) (end 151.945 61.715) (width 0.25) (layer B.Cu) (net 6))
 (segment (start 160.034 63.405) (end 153.635 63.405) (width 0.25) (layer B.Cu) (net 6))
 (via (at 162.6765 62.286498) (size 0.45) (drill 0.2) (layers F.Cu B.Cu) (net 5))
 (segment (start 162.4265 57.099) (end 162.964999 57.637499) (width 0.25) (layer F.Cu) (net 5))
 (segment (start 162.1065 57.099) (end 162.4265 57.099) (width 0.25) (layer F.Cu) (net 5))
 (segment (start 162.964999 57.637499) (end 162.964999 61.997999) (width 0.25) (layer F.Cu) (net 5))
 (segment (start 162.964999 61.997999) (end 162.6765 62.286498) (width 0.25) (layer F.Cu) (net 5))
 (segment (start 162.6765 62.2865) (end 162.6765 62.286498) (width 0.25) (layer B.Cu) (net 5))
 (segment (start 151.945 64.255) (end 160.708 64.255) (width 0.25) (layer B.Cu) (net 5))
 (segment (start 160.708 64.255) (end 162.6765 62.2865) (width 0.25) (layer B.Cu) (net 5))
 (segment (start 160.5175 64.763) (end 160.5175 64.763) (width 0.25) (layer F.Cu) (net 4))
 (via (at 160.526397 64.80501) (size 0.45) (drill 0.2) (layers F.Cu B.Cu) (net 4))
 (segment (start 162.1065 63.224907) (end 160.526397 64.80501) (width 0.25) (layer F.Cu) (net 4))
 (segment (start 151.945 66.795) (end 158.536407 66.795) (width 0.25) (layer B.Cu) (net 4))
 (segment (start 162.1065 61.244) (end 162.1065 63.224907) (width 0.25) (layer F.Cu) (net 4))
 (segment (start 158.536407 66.795) (end 160.526397 64.80501) (width 0.25) (layer B.Cu) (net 4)))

